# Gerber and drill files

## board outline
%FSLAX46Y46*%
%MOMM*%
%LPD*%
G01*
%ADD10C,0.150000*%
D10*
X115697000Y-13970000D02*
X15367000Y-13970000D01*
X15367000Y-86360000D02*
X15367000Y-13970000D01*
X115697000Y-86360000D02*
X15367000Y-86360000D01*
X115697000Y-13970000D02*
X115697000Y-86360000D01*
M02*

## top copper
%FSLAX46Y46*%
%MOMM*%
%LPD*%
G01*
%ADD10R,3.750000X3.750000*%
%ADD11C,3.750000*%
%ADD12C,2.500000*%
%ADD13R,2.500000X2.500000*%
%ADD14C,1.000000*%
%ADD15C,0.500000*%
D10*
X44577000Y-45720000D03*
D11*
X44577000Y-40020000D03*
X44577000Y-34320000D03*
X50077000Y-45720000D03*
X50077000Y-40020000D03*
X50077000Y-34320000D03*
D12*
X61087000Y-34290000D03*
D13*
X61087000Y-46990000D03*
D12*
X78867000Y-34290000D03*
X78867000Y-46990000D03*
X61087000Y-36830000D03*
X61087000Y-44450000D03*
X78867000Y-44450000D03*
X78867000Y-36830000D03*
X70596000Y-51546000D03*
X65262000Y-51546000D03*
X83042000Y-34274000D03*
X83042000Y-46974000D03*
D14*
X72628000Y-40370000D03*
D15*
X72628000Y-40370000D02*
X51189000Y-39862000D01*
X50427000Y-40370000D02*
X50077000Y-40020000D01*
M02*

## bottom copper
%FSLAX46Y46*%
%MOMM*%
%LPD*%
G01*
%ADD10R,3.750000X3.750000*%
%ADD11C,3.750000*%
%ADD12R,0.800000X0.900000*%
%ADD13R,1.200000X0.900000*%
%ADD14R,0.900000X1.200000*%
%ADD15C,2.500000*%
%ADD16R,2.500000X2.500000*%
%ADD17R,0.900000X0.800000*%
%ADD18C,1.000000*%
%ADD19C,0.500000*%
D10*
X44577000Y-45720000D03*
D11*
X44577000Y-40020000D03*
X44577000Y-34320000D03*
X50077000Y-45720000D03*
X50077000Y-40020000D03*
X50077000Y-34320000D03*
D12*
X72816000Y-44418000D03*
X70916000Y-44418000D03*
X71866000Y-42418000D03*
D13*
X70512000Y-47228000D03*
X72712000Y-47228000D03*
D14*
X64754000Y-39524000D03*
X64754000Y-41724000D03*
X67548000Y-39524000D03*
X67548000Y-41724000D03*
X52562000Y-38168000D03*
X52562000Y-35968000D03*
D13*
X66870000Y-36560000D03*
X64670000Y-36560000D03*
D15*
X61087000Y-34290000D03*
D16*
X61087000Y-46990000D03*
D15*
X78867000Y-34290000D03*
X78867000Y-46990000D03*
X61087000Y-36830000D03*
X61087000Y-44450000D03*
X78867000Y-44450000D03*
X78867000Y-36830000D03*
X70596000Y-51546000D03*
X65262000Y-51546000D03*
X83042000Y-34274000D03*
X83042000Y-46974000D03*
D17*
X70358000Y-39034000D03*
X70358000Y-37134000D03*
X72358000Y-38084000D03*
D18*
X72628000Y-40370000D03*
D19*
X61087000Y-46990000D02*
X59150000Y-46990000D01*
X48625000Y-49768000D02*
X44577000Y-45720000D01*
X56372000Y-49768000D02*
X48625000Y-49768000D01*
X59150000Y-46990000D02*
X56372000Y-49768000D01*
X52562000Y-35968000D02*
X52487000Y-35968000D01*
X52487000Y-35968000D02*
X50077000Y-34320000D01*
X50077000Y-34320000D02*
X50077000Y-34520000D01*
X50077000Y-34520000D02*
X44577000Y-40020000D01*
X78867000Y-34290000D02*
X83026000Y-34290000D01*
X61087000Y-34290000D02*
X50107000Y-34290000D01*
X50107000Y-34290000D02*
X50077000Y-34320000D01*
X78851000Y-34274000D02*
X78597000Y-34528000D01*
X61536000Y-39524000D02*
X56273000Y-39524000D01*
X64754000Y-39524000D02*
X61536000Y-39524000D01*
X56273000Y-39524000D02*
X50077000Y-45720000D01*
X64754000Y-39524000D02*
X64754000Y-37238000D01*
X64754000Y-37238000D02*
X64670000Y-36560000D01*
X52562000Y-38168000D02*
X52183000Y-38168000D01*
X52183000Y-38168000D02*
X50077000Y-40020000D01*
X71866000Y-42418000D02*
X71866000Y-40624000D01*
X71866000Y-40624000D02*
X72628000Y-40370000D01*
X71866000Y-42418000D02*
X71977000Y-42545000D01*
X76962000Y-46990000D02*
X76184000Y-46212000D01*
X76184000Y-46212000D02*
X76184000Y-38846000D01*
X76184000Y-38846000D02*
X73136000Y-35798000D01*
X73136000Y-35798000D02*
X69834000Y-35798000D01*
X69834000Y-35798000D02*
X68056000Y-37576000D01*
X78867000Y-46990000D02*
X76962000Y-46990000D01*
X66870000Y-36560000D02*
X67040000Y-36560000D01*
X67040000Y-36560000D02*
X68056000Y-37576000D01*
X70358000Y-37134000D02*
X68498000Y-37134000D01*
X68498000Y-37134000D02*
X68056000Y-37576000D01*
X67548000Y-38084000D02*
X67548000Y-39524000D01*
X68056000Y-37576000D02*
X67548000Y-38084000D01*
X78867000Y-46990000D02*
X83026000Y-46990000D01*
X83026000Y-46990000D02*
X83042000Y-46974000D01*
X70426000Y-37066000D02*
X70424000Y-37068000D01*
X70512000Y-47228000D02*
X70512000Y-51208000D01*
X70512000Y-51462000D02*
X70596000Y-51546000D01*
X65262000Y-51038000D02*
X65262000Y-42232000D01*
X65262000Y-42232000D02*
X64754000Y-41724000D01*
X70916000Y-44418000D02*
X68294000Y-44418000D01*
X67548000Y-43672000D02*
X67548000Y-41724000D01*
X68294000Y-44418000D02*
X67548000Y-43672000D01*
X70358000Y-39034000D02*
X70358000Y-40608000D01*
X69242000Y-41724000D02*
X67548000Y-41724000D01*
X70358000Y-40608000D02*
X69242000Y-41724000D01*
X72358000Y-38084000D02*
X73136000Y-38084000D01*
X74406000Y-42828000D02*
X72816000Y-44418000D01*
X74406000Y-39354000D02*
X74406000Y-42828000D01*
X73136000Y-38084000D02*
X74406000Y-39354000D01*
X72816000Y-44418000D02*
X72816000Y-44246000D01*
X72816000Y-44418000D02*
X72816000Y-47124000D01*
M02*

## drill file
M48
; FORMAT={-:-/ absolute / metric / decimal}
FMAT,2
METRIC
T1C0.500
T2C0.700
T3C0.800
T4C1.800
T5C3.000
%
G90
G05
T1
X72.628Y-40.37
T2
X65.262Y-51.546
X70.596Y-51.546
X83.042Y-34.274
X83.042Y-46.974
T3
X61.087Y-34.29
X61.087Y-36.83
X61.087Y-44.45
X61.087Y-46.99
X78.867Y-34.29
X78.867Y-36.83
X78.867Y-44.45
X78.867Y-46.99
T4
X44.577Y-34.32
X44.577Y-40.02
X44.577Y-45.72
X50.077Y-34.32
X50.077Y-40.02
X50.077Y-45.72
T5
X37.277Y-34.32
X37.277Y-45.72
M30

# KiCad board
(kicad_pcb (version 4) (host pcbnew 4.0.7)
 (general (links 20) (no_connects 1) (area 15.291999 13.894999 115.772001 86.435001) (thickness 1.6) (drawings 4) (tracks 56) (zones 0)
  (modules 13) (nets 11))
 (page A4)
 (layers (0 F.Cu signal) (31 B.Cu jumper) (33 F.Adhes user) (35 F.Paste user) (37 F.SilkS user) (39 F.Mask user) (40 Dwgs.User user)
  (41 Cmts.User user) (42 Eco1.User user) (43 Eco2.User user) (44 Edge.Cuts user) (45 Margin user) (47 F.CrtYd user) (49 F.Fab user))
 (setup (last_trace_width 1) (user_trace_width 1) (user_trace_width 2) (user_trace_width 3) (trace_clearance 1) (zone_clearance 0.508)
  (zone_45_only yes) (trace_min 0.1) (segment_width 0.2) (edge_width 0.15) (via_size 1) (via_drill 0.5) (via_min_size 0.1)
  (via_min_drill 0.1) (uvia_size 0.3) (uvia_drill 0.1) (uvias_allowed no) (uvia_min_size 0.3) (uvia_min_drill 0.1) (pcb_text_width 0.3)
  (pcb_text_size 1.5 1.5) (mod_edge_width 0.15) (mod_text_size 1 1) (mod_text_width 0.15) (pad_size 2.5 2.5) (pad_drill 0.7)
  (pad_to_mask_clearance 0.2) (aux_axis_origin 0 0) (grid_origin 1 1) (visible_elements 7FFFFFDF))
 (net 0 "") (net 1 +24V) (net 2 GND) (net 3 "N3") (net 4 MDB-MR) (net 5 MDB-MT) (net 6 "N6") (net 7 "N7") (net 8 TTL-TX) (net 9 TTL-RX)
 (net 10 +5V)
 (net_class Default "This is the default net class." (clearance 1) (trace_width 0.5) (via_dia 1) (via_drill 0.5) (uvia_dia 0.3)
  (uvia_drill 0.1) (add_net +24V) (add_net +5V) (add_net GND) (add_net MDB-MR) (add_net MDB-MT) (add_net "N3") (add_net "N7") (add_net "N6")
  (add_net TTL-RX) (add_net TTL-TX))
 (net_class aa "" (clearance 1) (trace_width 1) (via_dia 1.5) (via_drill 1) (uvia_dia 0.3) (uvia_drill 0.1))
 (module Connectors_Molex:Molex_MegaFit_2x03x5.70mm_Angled (layer F.Cu) (at 44.577 45.72 90)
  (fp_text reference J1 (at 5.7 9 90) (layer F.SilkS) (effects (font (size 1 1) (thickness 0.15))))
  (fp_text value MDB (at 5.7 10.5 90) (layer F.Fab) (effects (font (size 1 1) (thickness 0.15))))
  (pad 1 thru_hole rect (at 0 0 90) (size 3.75 3.75) (drill 1.8) (layers *.Cu *.Mask) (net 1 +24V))
  (pad 2 thru_hole circle (at 5.7 0 90) (size 3.75 3.75) (drill 1.8) (layers *.Cu *.Mask) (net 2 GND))
  (pad 3 thru_hole circle (at 11.4 0 90) (size 3.75 3.75) (drill 1.8) (layers *.Cu *.Mask) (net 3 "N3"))
  (pad 4 thru_hole circle (at 0 5.5 90) (size 3.75 3.75) (drill 1.8) (layers *.Cu *.Mask) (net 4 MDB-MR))
  (pad 5 thru_hole circle (at 5.7 5.5 90) (size 3.75 3.75) (drill 1.8) (layers *.Cu *.Mask) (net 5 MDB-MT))
  (pad 6 thru_hole circle (at 11.4 5.5 90) (size 3.75 3.75) (drill 1.8) (layers *.Cu *.Mask) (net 2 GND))
  (pad "" np_thru_hole circle (at 0 -7.3 90) (size 3 3) (drill 3) (layers *.Cu *.Mask))
  (pad "" np_thru_hole circle (at 11.4 -7.3 90) (size 3 3) (drill 3) (layers *.Cu *.Mask)))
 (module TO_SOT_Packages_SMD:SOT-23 (layer B.Cu) (at 71.866 43.418 90)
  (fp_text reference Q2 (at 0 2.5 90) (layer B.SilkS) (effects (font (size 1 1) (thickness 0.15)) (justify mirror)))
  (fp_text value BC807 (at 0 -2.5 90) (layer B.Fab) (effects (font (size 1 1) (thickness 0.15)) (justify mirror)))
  (pad 1 smd rect (at -1 0.95 90) (size 0.9 0.8) (layers B.Cu) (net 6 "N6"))
  (pad 2 smd rect (at -1 -0.95 90) (size 0.9 0.8) (layers B.Cu) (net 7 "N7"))
  (pad 3 smd rect (at 1 0 90) (size 0.9 0.8) (layers B.Cu) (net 5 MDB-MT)))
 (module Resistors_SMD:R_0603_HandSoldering (layer B.Cu) (at 71.612 47.228)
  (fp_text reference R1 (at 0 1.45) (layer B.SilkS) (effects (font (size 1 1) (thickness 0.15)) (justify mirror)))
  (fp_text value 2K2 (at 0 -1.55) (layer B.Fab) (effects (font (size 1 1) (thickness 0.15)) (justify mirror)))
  (pad 1 smd rect (at -1.1 0) (size 1.2 0.9) (layers B.Cu) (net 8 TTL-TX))
  (pad 2 smd rect (at 1.1 0) (size 1.2 0.9) (layers B.Cu) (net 6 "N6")))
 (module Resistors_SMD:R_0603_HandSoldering (layer B.Cu) (at 64.754 40.624 270)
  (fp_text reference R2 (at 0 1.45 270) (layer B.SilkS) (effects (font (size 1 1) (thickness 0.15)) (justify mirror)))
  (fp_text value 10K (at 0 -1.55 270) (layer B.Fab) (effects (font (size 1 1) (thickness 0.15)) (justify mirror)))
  (pad 1 smd rect (at -1.1 0 270) (size 1.2 0.9) (layers B.Cu) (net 4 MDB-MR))
  (pad 2 smd rect (at 1.1 0 270) (size 1.2 0.9) (layers B.Cu) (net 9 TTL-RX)))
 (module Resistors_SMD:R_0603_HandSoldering (layer B.Cu) (at 67.548 40.624 270)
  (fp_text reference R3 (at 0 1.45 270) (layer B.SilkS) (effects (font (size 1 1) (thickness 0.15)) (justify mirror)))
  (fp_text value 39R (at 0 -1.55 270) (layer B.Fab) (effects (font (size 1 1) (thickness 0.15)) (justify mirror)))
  (pad 1 smd rect (at -1.1 0 270) (size 1.2 0.9) (layers B.Cu) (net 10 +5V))
  (pad 2 smd rect (at 1.1 0 270) (size 1.2 0.9) (layers B.Cu) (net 7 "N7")))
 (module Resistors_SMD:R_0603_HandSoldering (layer B.Cu) (at 52.562 37.068 90)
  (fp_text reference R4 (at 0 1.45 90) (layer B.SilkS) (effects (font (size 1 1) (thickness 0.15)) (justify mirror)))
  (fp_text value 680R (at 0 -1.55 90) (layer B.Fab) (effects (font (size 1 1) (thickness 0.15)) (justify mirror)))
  (pad 1 smd rect (at -1.1 0 90) (size 1.2 0.9) (layers B.Cu) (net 5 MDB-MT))
  (pad 2 smd rect (at 1.1 0 90) (size 1.2 0.9) (layers B.Cu) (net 2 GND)))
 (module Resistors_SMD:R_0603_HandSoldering (layer B.Cu) (at 65.77 36.56 180)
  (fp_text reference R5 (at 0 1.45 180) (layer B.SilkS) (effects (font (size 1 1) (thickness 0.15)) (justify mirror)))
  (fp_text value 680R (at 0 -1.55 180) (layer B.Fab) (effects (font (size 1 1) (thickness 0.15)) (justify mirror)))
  (pad 1 smd rect (at -1.1 0 180) (size 1.2 0.9) (layers B.Cu) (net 10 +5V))
  (pad 2 smd rect (at 1.1 0 180) (size 1.2 0.9) (layers B.Cu) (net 4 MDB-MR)))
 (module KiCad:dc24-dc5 (layer F.Cu) (at 69.977 40.64)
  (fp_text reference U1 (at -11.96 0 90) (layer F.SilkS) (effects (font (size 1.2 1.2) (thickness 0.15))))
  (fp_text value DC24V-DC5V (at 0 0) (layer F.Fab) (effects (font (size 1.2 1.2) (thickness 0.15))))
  (pad 2 thru_hole circle (at -8.89 -6.35) (size 2.5 2.5) (drill 0.8) (layers *.Cu *.Mask) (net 2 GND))
  (pad 1 thru_hole rect (at -8.89 6.35) (size 2.5 2.5) (drill 0.8) (layers *.Cu *.Mask) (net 1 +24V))
  (pad 3 thru_hole circle (at 8.89 -6.35) (size 2.5 2.5) (drill 0.8) (layers *.Cu *.Mask) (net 2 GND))
  (pad 4 thru_hole circle (at 8.89 6.35) (size 2.5 2.5) (drill 0.8) (layers *.Cu *.Mask) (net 10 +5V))
  (pad 2.1 thru_hole circle (at -8.89 -3.81) (size 2.5 2.5) (drill 0.8) (layers *.Cu *.Mask))
  (pad 1.1 thru_hole circle (at -8.89 3.81) (size 2.5 2.5) (drill 0.8) (layers *.Cu *.Mask))
  (pad 4.1 thru_hole circle (at 8.89 3.81) (size 2.5 2.5) (drill 0.8) (layers *.Cu *.Mask))
  (pad 3.1 thru_hole circle (at 8.89 -3.81) (size 2.5 2.5) (drill 0.8) (layers *.Cu *.Mask)))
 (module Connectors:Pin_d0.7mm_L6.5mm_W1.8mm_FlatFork (layer F.Cu) (at 70.596 51.546)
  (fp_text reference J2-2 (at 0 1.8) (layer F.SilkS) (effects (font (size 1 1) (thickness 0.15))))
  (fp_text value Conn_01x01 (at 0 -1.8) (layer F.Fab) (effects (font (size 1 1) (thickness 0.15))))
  (pad 1 thru_hole circle (at 0 0) (size 2.5 2.5) (drill 0.7) (layers *.Cu *.Mask) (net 8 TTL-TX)))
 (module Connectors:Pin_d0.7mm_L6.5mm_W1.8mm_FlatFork (layer F.Cu) (at 65.262 51.546)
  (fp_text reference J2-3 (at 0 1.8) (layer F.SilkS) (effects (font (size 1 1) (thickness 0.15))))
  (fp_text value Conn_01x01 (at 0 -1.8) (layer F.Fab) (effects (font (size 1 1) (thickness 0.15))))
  (pad 1 thru_hole circle (at 0 0) (size 2.5 2.5) (drill 0.7) (layers *.Cu *.Mask) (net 9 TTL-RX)))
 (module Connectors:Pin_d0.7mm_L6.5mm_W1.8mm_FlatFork (layer F.Cu) (at 83.042 34.274)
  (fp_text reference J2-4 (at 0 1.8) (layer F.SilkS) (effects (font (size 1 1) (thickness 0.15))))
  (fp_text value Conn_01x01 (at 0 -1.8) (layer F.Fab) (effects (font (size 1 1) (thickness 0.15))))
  (pad 1 thru_hole circle (at 0 0) (size 2.5 2.5) (drill 0.7) (layers *.Cu *.Mask) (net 2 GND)))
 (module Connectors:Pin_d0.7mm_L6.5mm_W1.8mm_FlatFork (layer F.Cu) (at 83.042 46.974)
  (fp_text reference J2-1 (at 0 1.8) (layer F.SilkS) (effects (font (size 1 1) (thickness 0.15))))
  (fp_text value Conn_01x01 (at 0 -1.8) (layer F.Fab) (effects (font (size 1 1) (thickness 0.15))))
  (pad 1 thru_hole circle (at 0 0) (size 2.5 2.5) (drill 0.7) (layers *.Cu *.Mask) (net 10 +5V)))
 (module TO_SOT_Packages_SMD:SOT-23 (layer B.Cu) (at 71.358 38.084)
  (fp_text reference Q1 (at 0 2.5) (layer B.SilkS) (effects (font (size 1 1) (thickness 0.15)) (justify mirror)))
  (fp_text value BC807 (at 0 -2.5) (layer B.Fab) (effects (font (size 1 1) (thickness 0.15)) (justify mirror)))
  (pad 1 smd rect (at -1 0.95) (size 0.9 0.8) (layers B.Cu) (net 7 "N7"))
  (pad 2 smd rect (at -1 -0.95) (size 0.9 0.8) (layers B.Cu) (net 10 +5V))
  (pad 3 smd rect (at 1 0) (size 0.9 0.8) (layers B.Cu) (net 6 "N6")))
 (gr_line (start 115.697 13.97) (end 15.367 13.97) (angle 90) (layer Edge.Cuts) (width 0.15))
 (gr_line (start 15.367 86.36) (end 15.367 13.97) (angle 90) (layer Edge.Cuts) (width 0.15))
 (gr_line (start 115.697 86.36) (end 15.367 86.36) (angle 90) (layer Edge.Cuts) (width 0.15))
 (gr_line (start 115.697 13.97) (end 115.697 86.36) (angle 90) (layer Edge.Cuts) (width 0.15))
 (segment (start 61.087 46.99) (end 59.15 46.99) (width 0.5) (layer B.Cu) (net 1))
 (segment (start 48.625 49.768) (end 44.577 45.72) (width 0.5) (layer B.Cu) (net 1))
 (segment (start 56.372 49.768) (end 48.625 49.768) (width 0.5) (layer B.Cu) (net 1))
 (segment (start 59.15 46.99) (end 56.372 49.768) (width 0.5) (layer B.Cu) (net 1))
 (segment (start 52.562 35.968) (end 52.487 35.968) (width 0.5) (layer B.Cu) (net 2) (status 30))
 (segment (start 52.487 35.968) (end 50.077 34.32) (width 0.5) (layer B.Cu) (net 2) (status 10))
 (segment (start 50.077 34.32) (end 50.077 34.52) (width 0.5) (layer B.Cu) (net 2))
 (segment (start 50.077 34.52) (end 44.577 40.02) (width 0.5) (layer B.Cu) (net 2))
 (segment (start 78.867 34.29) (end 83.026 34.29) (width 0.5) (layer B.Cu) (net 2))
 (segment (start 61.087 34.29) (end 50.107 34.29) (width 0.5) (layer B.Cu) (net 2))
 (segment (start 50.107 34.29) (end 50.077 34.32) (width 0.5) (layer B.Cu) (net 2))
 (segment (start 78.851 34.274) (end 78.597 34.528) (width 0.5) (layer B.Cu) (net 2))
 (segment (start 61.536 39.524) (end 56.273 39.524) (width 0.5) (layer B.Cu) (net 4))
 (segment (start 64.754 39.524) (end 61.536 39.524) (width 0.5) (layer B.Cu) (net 4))
 (segment (start 56.273 39.524) (end 50.077 45.72) (width 0.5) (layer B.Cu) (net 4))
 (segment (start 64.754 39.524) (end 64.754 37.238) (width 0.5) (layer B.Cu) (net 4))
 (segment (start 64.754 37.238) (end 64.67 36.56) (width 0.5) (layer B.Cu) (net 4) (status 20))
 (segment (start 52.562 38.168) (end 52.183 38.168) (width 0.5) (layer B.Cu) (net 5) (status 30))
 (segment (start 52.183 38.168) (end 50.077 40.02) (width 0.5) (layer B.Cu) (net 5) (status 10))
 (segment (start 72.628 40.37) (end 51.189 39.862) (width 0.5) (layer F.Cu) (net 5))
 (segment (start 50.427 40.37) (end 50.077 40.02) (width 0.5) (layer F.Cu) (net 5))
 (segment (start 71.866 42.418) (end 71.866 40.624) (width 0.5) (layer B.Cu) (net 5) (status 10))
 (via (at 72.628 40.37) (size 1) (drill 0.5) (layers F.Cu B.Cu) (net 5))
 (segment (start 71.866 40.624) (end 72.628 40.37) (width 0.5) (layer B.Cu) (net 5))
 (segment (start 71.866 42.418) (end 71.977 42.545) (width 0.5) (layer B.Cu) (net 5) (status 30))
 (segment (start 76.962 46.99) (end 76.184 46.212) (width 0.5) (layer B.Cu) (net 10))
 (segment (start 76.184 46.212) (end 76.184 38.846) (width 0.5) (layer B.Cu) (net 10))
 (segment (start 76.184 38.846) (end 73.136 35.798) (width 0.5) (layer B.Cu) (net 10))
 (segment (start 73.136 35.798) (end 69.834 35.798) (width 0.5) (layer B.Cu) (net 10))
 (segment (start 69.834 35.798) (end 68.056 37.576) (width 0.5) (layer B.Cu) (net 10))
 (segment (start 78.867 46.99) (end 76.962 46.99) (width 0.5) (layer B.Cu) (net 10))
 (segment (start 66.87 36.56) (end 67.04 36.56) (width 0.5) (layer B.Cu) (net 10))
 (segment (start 67.04 36.56) (end 68.056 37.576) (width 0.5) (layer B.Cu) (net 10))
 (segment (start 70.358 37.134) (end 68.498 37.134) (width 0.5) (layer B.Cu) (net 10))
 (segment (start 68.498 37.134) (end 68.056 37.576) (width 0.5) (layer B.Cu) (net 10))
 (segment (start 67.548 38.084) (end 67.548 39.524) (width 0.5) (layer B.Cu) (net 10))
 (segment (start 68.056 37.576) (end 67.548 38.084) (width 0.5) (layer B.Cu) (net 10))
 (segment (start 78.867 46.99) (end 83.026 46.99) (width 0.5) (layer B.Cu) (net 10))
 (segment (start 83.026 46.99) (end 83.042 46.974) (width 0.5) (layer B.Cu) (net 10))
 (segment (start 70.426 37.066) (end 70.424 37.068) (width 0.5) (layer B.Cu) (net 10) (status 30))
 (segment (start 70.512 47.228) (end 70.512 51.208) (width 0.5) (layer B.Cu) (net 8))
 (segment (start 70.512 51.462) (end 70.596 51.546) (width 0.5) (layer B.Cu) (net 8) (status 30))
 (segment (start 65.262 51.038) (end 65.262 42.232) (width 0.5) (layer B.Cu) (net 9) (status 10))
 (segment (start 65.262 42.232) (end 64.754 41.724) (width 0.5) (layer B.Cu) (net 9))
 (segment (start 70.916 44.418) (end 68.294 44.418) (width 0.5) (layer B.Cu) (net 7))
 (segment (start 67.548 43.672) (end 67.548 41.724) (width 0.5) (layer B.Cu) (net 7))
 (segment (start 68.294 44.418) (end 67.548 43.672) (width 0.5) (layer B.Cu) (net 7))
 (segment (start 70.358 39.034) (end 70.358 40.608) (width 0.5) (layer B.Cu) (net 7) (status 10))
 (segment (start 69.242 41.724) (end 67.548 41.724) (width 0.5) (layer B.Cu) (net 7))
 (segment (start 70.358 40.608) (end 69.242 41.724) (width 0.5) (layer B.Cu) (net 7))
 (segment (start 72.358 38.084) (end 73.136 38.084) (width 0.5) (layer B.Cu) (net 6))
 (segment (start 74.406 42.828) (end 72.816 44.418) (width 0.5) (layer B.Cu) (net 6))
 (segment (start 74.406 39.354) (end 74.406 42.828) (width 0.5) (layer B.Cu) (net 6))
 (segment (start 73.136 38.084) (end 74.406 39.354) (width 0.5) (layer B.Cu) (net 6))
 (segment (start 72.816 44.418) (end 72.816 44.246) (width 0.5) (layer B.Cu) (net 6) (status 30))
 (segment (start 72.816 44.418) (end 72.816 47.124) (width 0.5) (layer B.Cu) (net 6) (status 10)))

